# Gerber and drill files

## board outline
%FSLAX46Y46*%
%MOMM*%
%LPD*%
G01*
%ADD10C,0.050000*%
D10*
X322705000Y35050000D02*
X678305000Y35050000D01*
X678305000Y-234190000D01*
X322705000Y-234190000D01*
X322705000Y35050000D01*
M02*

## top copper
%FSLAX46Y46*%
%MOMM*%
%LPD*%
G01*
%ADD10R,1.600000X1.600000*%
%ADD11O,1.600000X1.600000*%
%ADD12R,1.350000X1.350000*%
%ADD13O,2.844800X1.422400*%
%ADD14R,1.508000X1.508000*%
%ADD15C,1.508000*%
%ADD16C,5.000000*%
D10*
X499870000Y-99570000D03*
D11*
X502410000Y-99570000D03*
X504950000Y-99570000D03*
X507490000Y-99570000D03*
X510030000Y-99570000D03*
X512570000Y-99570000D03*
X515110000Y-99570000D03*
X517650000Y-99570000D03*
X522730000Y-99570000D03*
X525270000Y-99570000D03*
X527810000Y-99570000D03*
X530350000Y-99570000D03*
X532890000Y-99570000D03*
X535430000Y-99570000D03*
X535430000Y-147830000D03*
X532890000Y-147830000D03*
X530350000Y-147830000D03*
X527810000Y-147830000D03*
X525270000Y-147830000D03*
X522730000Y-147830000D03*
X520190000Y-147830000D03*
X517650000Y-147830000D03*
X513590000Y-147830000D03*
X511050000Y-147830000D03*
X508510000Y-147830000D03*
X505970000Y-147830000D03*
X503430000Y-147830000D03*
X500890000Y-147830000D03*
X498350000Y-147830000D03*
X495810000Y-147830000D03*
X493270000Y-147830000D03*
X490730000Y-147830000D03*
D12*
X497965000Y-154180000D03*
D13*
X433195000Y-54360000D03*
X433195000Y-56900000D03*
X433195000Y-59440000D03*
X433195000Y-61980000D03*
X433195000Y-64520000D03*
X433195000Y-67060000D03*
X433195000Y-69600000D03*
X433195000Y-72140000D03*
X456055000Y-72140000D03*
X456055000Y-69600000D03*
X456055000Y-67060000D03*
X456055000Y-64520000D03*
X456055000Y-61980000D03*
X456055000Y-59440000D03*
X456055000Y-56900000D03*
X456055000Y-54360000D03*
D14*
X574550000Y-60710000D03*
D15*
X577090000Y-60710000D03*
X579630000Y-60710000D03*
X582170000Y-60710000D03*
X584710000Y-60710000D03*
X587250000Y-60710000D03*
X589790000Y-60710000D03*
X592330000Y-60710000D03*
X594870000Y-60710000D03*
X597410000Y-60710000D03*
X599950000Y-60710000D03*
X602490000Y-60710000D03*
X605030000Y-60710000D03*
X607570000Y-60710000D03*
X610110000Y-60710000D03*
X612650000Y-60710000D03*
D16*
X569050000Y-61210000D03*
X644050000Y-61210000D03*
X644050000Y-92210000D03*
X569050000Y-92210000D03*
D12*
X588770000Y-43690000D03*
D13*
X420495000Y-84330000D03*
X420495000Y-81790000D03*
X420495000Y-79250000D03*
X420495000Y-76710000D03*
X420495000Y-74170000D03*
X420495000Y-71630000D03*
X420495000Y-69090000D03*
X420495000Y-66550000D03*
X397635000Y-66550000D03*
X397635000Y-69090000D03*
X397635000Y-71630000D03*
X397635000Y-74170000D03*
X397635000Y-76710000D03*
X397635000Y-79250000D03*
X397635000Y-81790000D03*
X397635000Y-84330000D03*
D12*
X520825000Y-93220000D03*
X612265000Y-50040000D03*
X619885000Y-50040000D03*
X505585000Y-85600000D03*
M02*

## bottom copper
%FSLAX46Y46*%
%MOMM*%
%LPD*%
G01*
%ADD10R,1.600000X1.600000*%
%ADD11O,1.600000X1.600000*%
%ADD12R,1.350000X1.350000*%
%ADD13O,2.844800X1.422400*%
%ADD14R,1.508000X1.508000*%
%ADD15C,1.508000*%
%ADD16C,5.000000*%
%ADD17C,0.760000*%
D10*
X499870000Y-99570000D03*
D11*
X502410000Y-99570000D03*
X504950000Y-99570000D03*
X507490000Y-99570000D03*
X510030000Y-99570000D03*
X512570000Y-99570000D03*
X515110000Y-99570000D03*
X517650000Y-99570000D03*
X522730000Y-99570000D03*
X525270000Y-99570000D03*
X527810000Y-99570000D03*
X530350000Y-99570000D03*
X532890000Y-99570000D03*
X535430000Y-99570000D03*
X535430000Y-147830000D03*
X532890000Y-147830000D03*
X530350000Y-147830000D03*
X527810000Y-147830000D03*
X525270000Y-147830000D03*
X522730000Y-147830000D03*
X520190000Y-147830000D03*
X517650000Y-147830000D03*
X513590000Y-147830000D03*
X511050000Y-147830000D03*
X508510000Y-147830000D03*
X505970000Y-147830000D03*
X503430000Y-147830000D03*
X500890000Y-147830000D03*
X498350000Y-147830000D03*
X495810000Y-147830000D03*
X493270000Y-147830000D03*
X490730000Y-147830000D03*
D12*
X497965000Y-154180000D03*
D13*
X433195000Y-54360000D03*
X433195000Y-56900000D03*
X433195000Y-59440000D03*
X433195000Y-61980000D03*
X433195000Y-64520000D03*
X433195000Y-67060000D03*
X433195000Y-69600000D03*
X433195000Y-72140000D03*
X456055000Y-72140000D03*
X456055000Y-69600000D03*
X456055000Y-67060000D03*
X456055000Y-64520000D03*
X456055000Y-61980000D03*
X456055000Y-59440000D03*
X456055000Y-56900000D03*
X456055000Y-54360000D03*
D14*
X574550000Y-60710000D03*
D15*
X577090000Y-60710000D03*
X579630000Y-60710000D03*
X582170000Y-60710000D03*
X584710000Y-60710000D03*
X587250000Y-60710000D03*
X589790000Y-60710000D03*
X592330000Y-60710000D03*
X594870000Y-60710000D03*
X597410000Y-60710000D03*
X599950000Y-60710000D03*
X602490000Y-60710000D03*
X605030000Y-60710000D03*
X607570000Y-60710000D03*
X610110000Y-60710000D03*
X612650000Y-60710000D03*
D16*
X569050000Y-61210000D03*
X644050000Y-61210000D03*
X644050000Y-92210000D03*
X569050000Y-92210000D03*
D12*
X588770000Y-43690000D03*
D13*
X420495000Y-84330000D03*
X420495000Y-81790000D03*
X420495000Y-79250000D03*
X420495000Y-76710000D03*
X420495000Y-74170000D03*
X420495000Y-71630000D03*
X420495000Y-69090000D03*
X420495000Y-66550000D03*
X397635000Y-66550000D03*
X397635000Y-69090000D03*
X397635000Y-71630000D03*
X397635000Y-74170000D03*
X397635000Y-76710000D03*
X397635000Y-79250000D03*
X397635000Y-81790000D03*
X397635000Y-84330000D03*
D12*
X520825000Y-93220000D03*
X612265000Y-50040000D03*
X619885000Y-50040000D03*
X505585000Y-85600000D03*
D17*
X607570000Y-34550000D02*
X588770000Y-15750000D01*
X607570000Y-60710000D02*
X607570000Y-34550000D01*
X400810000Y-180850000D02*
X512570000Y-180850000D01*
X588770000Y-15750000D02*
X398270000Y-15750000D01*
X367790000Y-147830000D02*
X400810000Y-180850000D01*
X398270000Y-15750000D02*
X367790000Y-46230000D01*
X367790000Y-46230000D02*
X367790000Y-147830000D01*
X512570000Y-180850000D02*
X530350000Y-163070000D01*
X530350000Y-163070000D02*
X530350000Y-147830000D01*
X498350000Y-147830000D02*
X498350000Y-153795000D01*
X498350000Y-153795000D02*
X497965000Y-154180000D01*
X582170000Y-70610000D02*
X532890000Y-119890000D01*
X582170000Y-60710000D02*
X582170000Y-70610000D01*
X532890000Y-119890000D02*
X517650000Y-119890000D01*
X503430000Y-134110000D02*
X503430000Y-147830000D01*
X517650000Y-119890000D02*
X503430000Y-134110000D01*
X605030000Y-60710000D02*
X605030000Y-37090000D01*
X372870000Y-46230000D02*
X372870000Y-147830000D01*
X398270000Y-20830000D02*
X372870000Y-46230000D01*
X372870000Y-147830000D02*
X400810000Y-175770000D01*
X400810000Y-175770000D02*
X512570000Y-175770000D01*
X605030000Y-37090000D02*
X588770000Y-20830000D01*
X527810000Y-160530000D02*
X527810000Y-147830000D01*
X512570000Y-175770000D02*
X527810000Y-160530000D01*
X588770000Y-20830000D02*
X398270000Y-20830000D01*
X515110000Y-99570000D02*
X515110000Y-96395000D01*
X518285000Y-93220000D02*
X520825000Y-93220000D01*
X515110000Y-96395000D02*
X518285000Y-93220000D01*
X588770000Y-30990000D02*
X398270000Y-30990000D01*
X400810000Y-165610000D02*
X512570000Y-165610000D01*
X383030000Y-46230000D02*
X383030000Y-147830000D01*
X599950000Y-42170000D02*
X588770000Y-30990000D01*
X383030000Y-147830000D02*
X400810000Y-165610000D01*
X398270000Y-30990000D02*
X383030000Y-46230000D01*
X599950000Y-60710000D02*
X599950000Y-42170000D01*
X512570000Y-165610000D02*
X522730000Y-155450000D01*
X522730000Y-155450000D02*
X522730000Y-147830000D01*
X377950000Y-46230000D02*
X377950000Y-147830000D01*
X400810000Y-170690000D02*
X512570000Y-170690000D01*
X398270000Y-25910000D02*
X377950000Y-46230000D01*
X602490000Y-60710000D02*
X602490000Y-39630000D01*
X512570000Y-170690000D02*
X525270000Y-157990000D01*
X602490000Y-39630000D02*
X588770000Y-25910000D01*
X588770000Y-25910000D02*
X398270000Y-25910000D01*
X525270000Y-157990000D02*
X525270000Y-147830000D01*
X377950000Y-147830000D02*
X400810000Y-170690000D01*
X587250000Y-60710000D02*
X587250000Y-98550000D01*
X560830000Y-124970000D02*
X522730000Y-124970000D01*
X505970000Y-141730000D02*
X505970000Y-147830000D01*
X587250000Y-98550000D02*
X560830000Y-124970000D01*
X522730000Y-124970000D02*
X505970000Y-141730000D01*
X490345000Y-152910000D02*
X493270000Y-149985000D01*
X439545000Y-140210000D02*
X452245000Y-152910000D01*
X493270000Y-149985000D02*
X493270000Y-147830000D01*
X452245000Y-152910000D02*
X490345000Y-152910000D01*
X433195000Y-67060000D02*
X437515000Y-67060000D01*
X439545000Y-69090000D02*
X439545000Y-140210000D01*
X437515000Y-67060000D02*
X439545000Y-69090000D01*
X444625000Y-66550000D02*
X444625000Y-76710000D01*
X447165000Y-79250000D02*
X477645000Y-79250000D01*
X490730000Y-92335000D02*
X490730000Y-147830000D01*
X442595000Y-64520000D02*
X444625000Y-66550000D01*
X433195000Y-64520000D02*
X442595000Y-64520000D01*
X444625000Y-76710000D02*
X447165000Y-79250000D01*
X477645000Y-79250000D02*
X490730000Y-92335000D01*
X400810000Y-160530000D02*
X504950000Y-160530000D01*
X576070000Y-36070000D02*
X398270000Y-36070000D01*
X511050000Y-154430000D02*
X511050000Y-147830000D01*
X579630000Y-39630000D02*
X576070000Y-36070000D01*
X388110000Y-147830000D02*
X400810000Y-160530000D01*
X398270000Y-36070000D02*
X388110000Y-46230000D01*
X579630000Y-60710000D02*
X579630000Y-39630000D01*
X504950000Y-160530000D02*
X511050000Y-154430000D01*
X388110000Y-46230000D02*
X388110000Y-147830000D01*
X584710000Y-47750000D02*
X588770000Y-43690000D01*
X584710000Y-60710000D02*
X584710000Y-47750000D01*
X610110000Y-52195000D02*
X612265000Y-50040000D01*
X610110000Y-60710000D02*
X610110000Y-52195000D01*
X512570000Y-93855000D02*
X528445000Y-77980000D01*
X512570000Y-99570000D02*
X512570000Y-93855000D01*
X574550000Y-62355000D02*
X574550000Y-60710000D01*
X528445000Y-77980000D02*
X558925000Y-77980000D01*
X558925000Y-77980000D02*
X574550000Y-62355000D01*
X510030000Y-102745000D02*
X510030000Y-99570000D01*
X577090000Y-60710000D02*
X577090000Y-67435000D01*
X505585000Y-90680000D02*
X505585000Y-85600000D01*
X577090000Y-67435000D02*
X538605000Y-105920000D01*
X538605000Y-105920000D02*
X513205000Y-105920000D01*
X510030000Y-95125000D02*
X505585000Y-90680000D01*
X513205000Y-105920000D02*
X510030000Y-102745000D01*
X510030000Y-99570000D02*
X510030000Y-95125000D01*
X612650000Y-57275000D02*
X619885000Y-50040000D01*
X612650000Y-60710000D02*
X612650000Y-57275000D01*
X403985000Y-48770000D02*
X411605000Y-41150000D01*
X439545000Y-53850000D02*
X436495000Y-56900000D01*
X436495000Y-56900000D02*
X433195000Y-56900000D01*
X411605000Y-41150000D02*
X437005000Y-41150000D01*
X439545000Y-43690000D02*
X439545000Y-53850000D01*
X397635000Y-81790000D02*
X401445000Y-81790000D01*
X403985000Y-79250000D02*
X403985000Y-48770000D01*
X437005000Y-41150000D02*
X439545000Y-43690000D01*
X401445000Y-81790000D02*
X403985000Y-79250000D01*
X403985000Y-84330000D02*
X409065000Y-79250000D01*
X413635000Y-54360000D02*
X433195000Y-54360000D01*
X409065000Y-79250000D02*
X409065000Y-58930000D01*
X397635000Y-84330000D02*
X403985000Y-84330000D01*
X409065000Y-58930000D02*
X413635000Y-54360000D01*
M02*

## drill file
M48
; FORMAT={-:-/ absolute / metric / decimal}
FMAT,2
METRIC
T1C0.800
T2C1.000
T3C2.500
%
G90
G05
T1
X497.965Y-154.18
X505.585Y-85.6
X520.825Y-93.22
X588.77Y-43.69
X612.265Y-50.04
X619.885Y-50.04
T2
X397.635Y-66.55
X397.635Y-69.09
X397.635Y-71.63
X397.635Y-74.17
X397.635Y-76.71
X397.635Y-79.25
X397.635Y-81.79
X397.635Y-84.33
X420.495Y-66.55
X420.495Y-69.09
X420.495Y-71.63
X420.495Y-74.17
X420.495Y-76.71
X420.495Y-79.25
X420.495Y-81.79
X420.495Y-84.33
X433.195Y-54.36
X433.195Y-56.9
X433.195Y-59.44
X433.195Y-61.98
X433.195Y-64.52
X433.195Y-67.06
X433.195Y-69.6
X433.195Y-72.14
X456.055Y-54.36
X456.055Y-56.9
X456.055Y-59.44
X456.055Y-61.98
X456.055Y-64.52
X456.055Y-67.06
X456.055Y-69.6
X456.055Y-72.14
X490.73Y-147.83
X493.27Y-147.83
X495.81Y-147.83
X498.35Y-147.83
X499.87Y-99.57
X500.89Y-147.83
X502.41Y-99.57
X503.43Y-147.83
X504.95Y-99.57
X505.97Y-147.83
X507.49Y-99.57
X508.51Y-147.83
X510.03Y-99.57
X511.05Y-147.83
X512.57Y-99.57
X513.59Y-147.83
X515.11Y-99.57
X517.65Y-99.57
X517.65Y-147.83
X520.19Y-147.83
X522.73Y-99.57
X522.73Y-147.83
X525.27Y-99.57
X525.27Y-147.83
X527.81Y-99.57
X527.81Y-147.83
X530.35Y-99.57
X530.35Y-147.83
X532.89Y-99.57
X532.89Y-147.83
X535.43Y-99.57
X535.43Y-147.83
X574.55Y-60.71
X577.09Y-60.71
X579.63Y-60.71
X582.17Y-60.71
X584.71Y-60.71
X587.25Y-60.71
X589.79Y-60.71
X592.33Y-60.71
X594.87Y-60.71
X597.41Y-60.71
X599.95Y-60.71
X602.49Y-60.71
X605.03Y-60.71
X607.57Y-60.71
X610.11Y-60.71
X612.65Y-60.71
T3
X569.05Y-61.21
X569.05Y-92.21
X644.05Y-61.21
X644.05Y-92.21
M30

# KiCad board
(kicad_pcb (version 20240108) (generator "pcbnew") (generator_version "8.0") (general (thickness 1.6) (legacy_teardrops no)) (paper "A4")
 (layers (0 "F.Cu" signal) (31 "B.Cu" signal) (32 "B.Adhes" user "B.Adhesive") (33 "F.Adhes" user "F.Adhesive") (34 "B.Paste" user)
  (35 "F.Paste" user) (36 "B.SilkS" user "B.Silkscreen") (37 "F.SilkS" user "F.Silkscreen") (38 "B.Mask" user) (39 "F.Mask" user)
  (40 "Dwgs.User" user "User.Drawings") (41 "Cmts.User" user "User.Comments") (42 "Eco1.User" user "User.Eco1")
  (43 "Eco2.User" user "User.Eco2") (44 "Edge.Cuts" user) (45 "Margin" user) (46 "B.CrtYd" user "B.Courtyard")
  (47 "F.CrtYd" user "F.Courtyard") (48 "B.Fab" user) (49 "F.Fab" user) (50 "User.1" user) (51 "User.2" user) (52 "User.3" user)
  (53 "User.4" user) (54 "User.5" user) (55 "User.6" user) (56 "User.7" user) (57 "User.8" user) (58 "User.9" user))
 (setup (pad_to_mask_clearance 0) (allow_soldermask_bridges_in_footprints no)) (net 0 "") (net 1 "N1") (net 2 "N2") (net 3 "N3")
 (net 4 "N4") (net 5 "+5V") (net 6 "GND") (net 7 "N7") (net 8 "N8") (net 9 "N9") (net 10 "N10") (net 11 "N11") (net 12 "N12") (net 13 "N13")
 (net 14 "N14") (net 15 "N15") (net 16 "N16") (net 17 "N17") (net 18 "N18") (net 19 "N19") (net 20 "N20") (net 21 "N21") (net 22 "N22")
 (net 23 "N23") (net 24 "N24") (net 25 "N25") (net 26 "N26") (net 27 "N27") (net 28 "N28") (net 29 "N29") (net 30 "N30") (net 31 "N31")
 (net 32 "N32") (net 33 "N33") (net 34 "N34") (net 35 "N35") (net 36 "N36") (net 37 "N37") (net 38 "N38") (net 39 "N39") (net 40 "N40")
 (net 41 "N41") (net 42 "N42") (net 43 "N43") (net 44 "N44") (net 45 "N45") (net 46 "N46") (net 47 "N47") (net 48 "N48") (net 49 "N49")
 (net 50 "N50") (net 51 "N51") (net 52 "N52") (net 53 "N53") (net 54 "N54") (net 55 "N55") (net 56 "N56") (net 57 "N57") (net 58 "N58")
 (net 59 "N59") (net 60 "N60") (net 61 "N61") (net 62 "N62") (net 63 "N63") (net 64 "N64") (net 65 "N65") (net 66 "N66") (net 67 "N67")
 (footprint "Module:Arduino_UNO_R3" (layer "F.Cu") (at 499.87 99.57)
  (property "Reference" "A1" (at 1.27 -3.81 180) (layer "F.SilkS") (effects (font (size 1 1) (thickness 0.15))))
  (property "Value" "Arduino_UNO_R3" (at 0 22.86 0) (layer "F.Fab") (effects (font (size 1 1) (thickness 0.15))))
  (pad "1" thru_hole rect (at 0 0 90) (size 1.6 1.6) (drill 1) (layers "*.Cu" "*.Mask") (remove_unused_layers no) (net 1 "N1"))
  (pad "2" thru_hole oval (at 2.54 0 90) (size 1.6 1.6) (drill 1) (layers "*.Cu" "*.Mask") (remove_unused_layers no) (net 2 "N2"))
  (pad "3" thru_hole oval (at 5.08 0 90) (size 1.6 1.6) (drill 1) (layers "*.Cu" "*.Mask") (remove_unused_layers no) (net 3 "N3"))
  (pad "4" thru_hole oval (at 7.62 0 90) (size 1.6 1.6) (drill 1) (layers "*.Cu" "*.Mask") (remove_unused_layers no) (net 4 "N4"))
  (pad "5" thru_hole oval (at 10.16 0 90) (size 1.6 1.6) (drill 1) (layers "*.Cu" "*.Mask") (remove_unused_layers no) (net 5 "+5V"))
  (pad "6" thru_hole oval (at 12.7 0 90) (size 1.6 1.6) (drill 1) (layers "*.Cu" "*.Mask") (remove_unused_layers no) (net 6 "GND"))
  (pad "7" thru_hole oval (at 15.24 0 90) (size 1.6 1.6) (drill 1) (layers "*.Cu" "*.Mask") (remove_unused_layers no) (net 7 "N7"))
  (pad "8" thru_hole oval (at 17.78 0 90) (size 1.6 1.6) (drill 1) (layers "*.Cu" "*.Mask") (remove_unused_layers no) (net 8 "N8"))
  (pad "9" thru_hole oval (at 22.86 0 90) (size 1.6 1.6) (drill 1) (layers "*.Cu" "*.Mask") (remove_unused_layers no) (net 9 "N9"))
  (pad "10" thru_hole oval (at 25.4 0 90) (size 1.6 1.6) (drill 1) (layers "*.Cu" "*.Mask") (remove_unused_layers no) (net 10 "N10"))
  (pad "11" thru_hole oval (at 27.94 0 90) (size 1.6 1.6) (drill 1) (layers "*.Cu" "*.Mask") (remove_unused_layers no) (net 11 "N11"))
  (pad "12" thru_hole oval (at 30.48 0 90) (size 1.6 1.6) (drill 1) (layers "*.Cu" "*.Mask") (remove_unused_layers no) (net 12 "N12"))
  (pad "13" thru_hole oval (at 33.02 0 90) (size 1.6 1.6) (drill 1) (layers "*.Cu" "*.Mask") (remove_unused_layers no) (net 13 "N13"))
  (pad "14" thru_hole oval (at 35.56 0 90) (size 1.6 1.6) (drill 1) (layers "*.Cu" "*.Mask") (remove_unused_layers no) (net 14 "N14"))
  (pad "15" thru_hole oval (at 35.56 48.26 90) (size 1.6 1.6) (drill 1) (layers "*.Cu" "*.Mask") (remove_unused_layers no) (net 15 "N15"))
  (pad "16" thru_hole oval (at 33.02 48.26 90) (size 1.6 1.6) (drill 1) (layers "*.Cu" "*.Mask") (remove_unused_layers no) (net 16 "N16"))
  (pad "17" thru_hole oval (at 30.48 48.26 90) (size 1.6 1.6) (drill 1) (layers "*.Cu" "*.Mask") (remove_unused_layers no) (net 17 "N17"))
  (pad "18" thru_hole oval (at 27.94 48.26 90) (size 1.6 1.6) (drill 1) (layers "*.Cu" "*.Mask") (remove_unused_layers no) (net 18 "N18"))
  (pad "19" thru_hole oval (at 25.4 48.26 90) (size 1.6 1.6) (drill 1) (layers "*.Cu" "*.Mask") (remove_unused_layers no) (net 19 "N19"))
  (pad "20" thru_hole oval (at 22.86 48.26 90) (size 1.6 1.6) (drill 1) (layers "*.Cu" "*.Mask") (remove_unused_layers no) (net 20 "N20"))
  (pad "21" thru_hole oval (at 20.32 48.26 90) (size 1.6 1.6) (drill 1) (layers "*.Cu" "*.Mask") (remove_unused_layers no) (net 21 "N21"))
  (pad "22" thru_hole oval (at 17.78 48.26 90) (size 1.6 1.6) (drill 1) (layers "*.Cu" "*.Mask") (remove_unused_layers no) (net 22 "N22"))
  (pad "23" thru_hole oval (at 13.72 48.26 90) (size 1.6 1.6) (drill 1) (layers "*.Cu" "*.Mask") (remove_unused_layers no) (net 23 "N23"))
  (pad "24" thru_hole oval (at 11.18 48.26 90) (size 1.6 1.6) (drill 1) (layers "*.Cu" "*.Mask") (remove_unused_layers no) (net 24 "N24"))
  (pad "25" thru_hole oval (at 8.64 48.26 90) (size 1.6 1.6) (drill 1) (layers "*.Cu" "*.Mask") (remove_unused_layers no) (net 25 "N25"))
  (pad "26" thru_hole oval (at 6.1 48.26 90) (size 1.6 1.6) (drill 1) (layers "*.Cu" "*.Mask") (remove_unused_layers no) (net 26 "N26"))
  (pad "27" thru_hole oval (at 3.56 48.26 90) (size 1.6 1.6) (drill 1) (layers "*.Cu" "*.Mask") (remove_unused_layers no) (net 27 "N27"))
  (pad "28" thru_hole oval (at 1.02 48.26 90) (size 1.6 1.6) (drill 1) (layers "*.Cu" "*.Mask") (remove_unused_layers no) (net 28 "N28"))
  (pad "29" thru_hole oval (at -1.52 48.26 90) (size 1.6 1.6) (drill 1) (layers "*.Cu" "*.Mask") (remove_unused_layers no) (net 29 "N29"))
  (pad "30" thru_hole oval (at -4.06 48.26 90) (size 1.6 1.6) (drill 1) (layers "*.Cu" "*.Mask") (remove_unused_layers no) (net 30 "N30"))
  (pad "31" thru_hole oval (at -6.6 48.26 90) (size 1.6 1.6) (drill 1) (layers "*.Cu" "*.Mask") (remove_unused_layers no) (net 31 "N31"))
  (pad "32" thru_hole oval (at -9.14 48.26 90) (size 1.6 1.6) (drill 1) (layers "*.Cu" "*.Mask") (remove_unused_layers no) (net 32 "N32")))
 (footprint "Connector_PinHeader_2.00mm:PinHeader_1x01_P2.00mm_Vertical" (layer "F.Cu") (at 497.965 154.18)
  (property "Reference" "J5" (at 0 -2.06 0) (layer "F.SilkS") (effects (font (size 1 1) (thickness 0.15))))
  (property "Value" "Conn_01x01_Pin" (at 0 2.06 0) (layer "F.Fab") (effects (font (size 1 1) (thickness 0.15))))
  (pad "1" thru_hole rect (at 0 0) (size 1.35 1.35) (drill 0.8) (layers "*.Cu" "*.Mask") (remove_unused_layers no) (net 29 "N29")))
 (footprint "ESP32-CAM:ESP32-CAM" (layer "F.Cu") (at 444.625 64.52)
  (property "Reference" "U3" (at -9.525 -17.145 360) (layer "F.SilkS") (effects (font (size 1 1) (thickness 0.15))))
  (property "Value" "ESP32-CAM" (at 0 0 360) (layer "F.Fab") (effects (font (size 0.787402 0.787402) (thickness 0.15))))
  (pad "P$1" thru_hole oval (at -11.43 -10.16) (size 2.8448 1.4224) (drill 1) (layers "*.Cu" "*.Mask") (remove_unused_layers no)
   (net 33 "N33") (solder_mask_margin 0.102))
  (pad "P$2" thru_hole oval (at -11.43 -7.62) (size 2.8448 1.4224) (drill 1) (layers "*.Cu" "*.Mask") (remove_unused_layers no)
   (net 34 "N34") (solder_mask_margin 0.102))
  (pad "P$3" thru_hole oval (at -11.43 -5.08) (size 2.8448 1.4224) (drill 1) (layers "*.Cu" "*.Mask") (remove_unused_layers no)
   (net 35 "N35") (solder_mask_margin 0.102))
  (pad "P$4" thru_hole oval (at -11.43 -2.54) (size 2.8448 1.4224) (drill 1) (layers "*.Cu" "*.Mask") (remove_unused_layers no)
   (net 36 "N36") (solder_mask_margin 0.102))
  (pad "P$5" thru_hole oval (at -11.43 0) (size 2.8448 1.4224) (drill 1) (layers "*.Cu" "*.Mask") (remove_unused_layers no) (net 32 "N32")
   (solder_mask_margin 0.102))
  (pad "P$6" thru_hole oval (at -11.43 2.54) (size 2.8448 1.4224) (drill 1) (layers "*.Cu" "*.Mask") (remove_unused_layers no)
   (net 31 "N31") (solder_mask_margin 0.102))
  (pad "P$7" thru_hole oval (at -11.43 5.08) (size 2.8448 1.4224) (drill 1) (layers "*.Cu" "*.Mask") (remove_unused_layers no)
   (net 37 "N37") (solder_mask_margin 0.102))
  (pad "P$8" thru_hole oval (at -11.43 7.62) (size 2.8448 1.4224) (drill 1) (layers "*.Cu" "*.Mask") (remove_unused_layers no)
   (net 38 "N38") (solder_mask_margin 0.102))
  (pad "P$9" thru_hole oval (at 11.43 7.62) (size 2.8448 1.4224) (drill 1) (layers "*.Cu" "*.Mask") (remove_unused_layers no) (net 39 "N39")
   (solder_mask_margin 0.102))
  (pad "P$10" thru_hole oval (at 11.43 5.08) (size 2.8448 1.4224) (drill 1) (layers "*.Cu" "*.Mask") (remove_unused_layers no)
   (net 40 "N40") (solder_mask_margin 0.102))
  (pad "P$11" thru_hole oval (at 11.43 2.54) (size 2.8448 1.4224) (drill 1) (layers "*.Cu" "*.Mask") (remove_unused_layers no)
   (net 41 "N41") (solder_mask_margin 0.102))
  (pad "P$12" thru_hole oval (at 11.43 0) (size 2.8448 1.4224) (drill 1) (layers "*.Cu" "*.Mask") (remove_unused_layers no) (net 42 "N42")
   (solder_mask_margin 0.102))
  (pad "P$13" thru_hole oval (at 11.43 -2.54) (size 2.8448 1.4224) (drill 1) (layers "*.Cu" "*.Mask") (remove_unused_layers no)
   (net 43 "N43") (solder_mask_margin 0.102))
  (pad "P$14" thru_hole oval (at 11.43 -5.08) (size 2.8448 1.4224) (drill 1) (layers "*.Cu" "*.Mask") (remove_unused_layers no)
   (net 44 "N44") (solder_mask_margin 0.102))
  (pad "P$15" thru_hole oval (at 11.43 -7.62) (size 2.8448 1.4224) (drill 1) (layers "*.Cu" "*.Mask") (remove_unused_layers no)
   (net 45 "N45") (solder_mask_margin 0.102))
  (pad "P$16" thru_hole oval (at 11.43 -10.16) (size 2.8448 1.4224) (drill 1) (layers "*.Cu" "*.Mask") (remove_unused_layers no)
   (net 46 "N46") (solder_mask_margin 0.102)))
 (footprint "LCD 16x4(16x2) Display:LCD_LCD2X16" (layer "F.Cu") (at 606.55 76.71)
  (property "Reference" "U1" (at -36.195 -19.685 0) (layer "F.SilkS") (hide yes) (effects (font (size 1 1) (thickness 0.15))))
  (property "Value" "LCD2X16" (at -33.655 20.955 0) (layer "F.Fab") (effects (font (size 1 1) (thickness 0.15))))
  (pad "1" thru_hole rect (at -32 -16) (size 1.508 1.508) (drill 1) (layers "*.Cu" "*.Mask") (remove_unused_layers no) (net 6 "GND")
   (solder_mask_margin 0.102))
  (pad "2" thru_hole circle (at -29.46 -16) (size 1.508 1.508) (drill 1) (layers "*.Cu" "*.Mask") (remove_unused_layers no) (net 5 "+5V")
   (solder_mask_margin 0.102))
  (pad "3" thru_hole circle (at -26.92 -16) (size 1.508 1.508) (drill 1) (layers "*.Cu" "*.Mask") (remove_unused_layers no) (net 24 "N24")
   (solder_mask_margin 0.102))
  (pad "4" thru_hole circle (at -24.38 -16) (size 1.508 1.508) (drill 1) (layers "*.Cu" "*.Mask") (remove_unused_layers no) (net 27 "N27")
   (solder_mask_margin 0.102))
  (pad "5" thru_hole circle (at -21.84 -16) (size 1.508 1.508) (drill 1) (layers "*.Cu" "*.Mask") (remove_unused_layers no) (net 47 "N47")
   (solder_mask_margin 0.102))
  (pad "6" thru_hole circle (at -19.3 -16) (size 1.508 1.508) (drill 1) (layers "*.Cu" "*.Mask") (remove_unused_layers no) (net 26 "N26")
   (solder_mask_margin 0.102))
  (pad "7" thru_hole circle (at -16.76 -16) (size 1.508 1.508) (drill 1) (layers "*.Cu" "*.Mask") (remove_unused_layers no) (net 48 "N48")
   (solder_mask_margin 0.102))
  (pad "8" thru_hole circle (at -14.22 -16) (size 1.508 1.508) (drill 1) (layers "*.Cu" "*.Mask") (remove_unused_layers no) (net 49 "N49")
   (solder_mask_margin 0.102))
  (pad "9" thru_hole circle (at -11.68 -16) (size 1.508 1.508) (drill 1) (layers "*.Cu" "*.Mask") (remove_unused_layers no) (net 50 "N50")
   (solder_mask_margin 0.102))
  (pad "10" thru_hole circle (at -9.14 -16) (size 1.508 1.508) (drill 1) (layers "*.Cu" "*.Mask") (remove_unused_layers no) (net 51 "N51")
   (solder_mask_margin 0.102))
  (pad "11" thru_hole circle (at -6.6 -16) (size 1.508 1.508) (drill 1) (layers "*.Cu" "*.Mask") (remove_unused_layers no) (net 20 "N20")
   (solder_mask_margin 0.102))
  (pad "12" thru_hole circle (at -4.06 -16) (size 1.508 1.508) (drill 1) (layers "*.Cu" "*.Mask") (remove_unused_layers no) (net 19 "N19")
   (solder_mask_margin 0.102))
  (pad "13" thru_hole circle (at -1.52 -16) (size 1.508 1.508) (drill 1) (layers "*.Cu" "*.Mask") (remove_unused_layers no) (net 18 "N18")
   (solder_mask_margin 0.102))
  (pad "14" thru_hole circle (at 1.02 -16) (size 1.508 1.508) (drill 1) (layers "*.Cu" "*.Mask") (remove_unused_layers no) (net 17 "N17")
   (solder_mask_margin 0.102))
  (pad "15" thru_hole circle (at 3.56 -16) (size 1.508 1.508) (drill 1) (layers "*.Cu" "*.Mask") (remove_unused_layers no) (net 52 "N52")
   (solder_mask_margin 0.102))
  (pad "16" thru_hole circle (at 6.1 -16) (size 1.508 1.508) (drill 1) (layers "*.Cu" "*.Mask") (remove_unused_layers no) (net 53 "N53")
   (solder_mask_margin 0.102))
  (pad "S1" thru_hole circle (at -37.5 -15.5) (size 5 5) (drill 2.5) (layers "*.Cu" "*.Mask") (remove_unused_layers no)
   (solder_mask_margin 0.102))
  (pad "S2" thru_hole circle (at 37.5 -15.5) (size 5 5) (drill 2.5) (layers "*.Cu" "*.Mask") (remove_unused_layers no)
   (solder_mask_margin 0.102))
  (pad "S3" thru_hole circle (at 37.5 15.5) (size 5 5) (drill 2.5) (layers "*.Cu" "*.Mask") (remove_unused_layers no)
   (solder_mask_margin 0.102))
  (pad "S4" thru_hole circle (at -37.5 15.5) (size 5 5) (drill 2.5) (layers "*.Cu" "*.Mask") (remove_unused_layers no)
   (solder_mask_margin 0.102)))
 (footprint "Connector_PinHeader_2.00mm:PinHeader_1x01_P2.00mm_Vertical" (layer "F.Cu") (at 588.77 43.69)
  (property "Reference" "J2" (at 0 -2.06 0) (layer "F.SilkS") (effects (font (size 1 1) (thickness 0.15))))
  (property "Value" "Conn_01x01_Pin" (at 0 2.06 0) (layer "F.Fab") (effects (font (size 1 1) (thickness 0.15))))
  (pad "1" thru_hole rect (at 0 0) (size 1.35 1.35) (drill 0.8) (layers "*.Cu" "*.Mask") (remove_unused_layers no) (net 47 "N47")))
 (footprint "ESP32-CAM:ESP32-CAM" (layer "F.Cu") (at 409.065 74.17 180)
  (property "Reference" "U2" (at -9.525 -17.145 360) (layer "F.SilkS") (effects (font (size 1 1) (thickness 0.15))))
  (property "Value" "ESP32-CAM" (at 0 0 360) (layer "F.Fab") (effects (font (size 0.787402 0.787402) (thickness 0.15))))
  (pad "P$1" thru_hole oval (at -11.43 -10.16 180) (size 2.8448 1.4224) (drill 1) (layers "*.Cu" "*.Mask") (remove_unused_layers no)
   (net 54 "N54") (solder_mask_margin 0.102))
  (pad "P$2" thru_hole oval (at -11.43 -7.62 180) (size 2.8448 1.4224) (drill 1) (layers "*.Cu" "*.Mask") (remove_unused_layers no)
   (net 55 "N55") (solder_mask_margin 0.102))
  (pad "P$3" thru_hole oval (at -11.43 -5.08 180) (size 2.8448 1.4224) (drill 1) (layers "*.Cu" "*.Mask") (remove_unused_layers no)
   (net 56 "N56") (solder_mask_margin 0.102))
  (pad "P$4" thru_hole oval (at -11.43 -2.54 180) (size 2.8448 1.4224) (drill 1) (layers "*.Cu" "*.Mask") (remove_unused_layers no)
   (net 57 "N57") (solder_mask_margin 0.102))
  (pad "P$5" thru_hole oval (at -11.43 0 180) (size 2.8448 1.4224) (drill 1) (layers "*.Cu" "*.Mask") (remove_unused_layers no)
   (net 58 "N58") (solder_mask_margin 0.102))
  (pad "P$6" thru_hole oval (at -11.43 2.54 180) (size 2.8448 1.4224) (drill 1) (layers "*.Cu" "*.Mask") (remove_unused_layers no)
   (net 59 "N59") (solder_mask_margin 0.102))
  (pad "P$7" thru_hole oval (at -11.43 5.08 180) (size 2.8448 1.4224) (drill 1) (layers "*.Cu" "*.Mask") (remove_unused_layers no)
   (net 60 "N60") (solder_mask_margin 0.102))
  (pad "P$8" thru_hole oval (at -11.43 7.62 180) (size 2.8448 1.4224) (drill 1) (layers "*.Cu" "*.Mask") (remove_unused_layers no)
   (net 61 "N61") (solder_mask_margin 0.102))
  (pad "P$9" thru_hole oval (at 11.43 7.62 180) (size 2.8448 1.4224) (drill 1) (layers "*.Cu" "*.Mask") (remove_unused_layers no)
   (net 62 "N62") (solder_mask_margin 0.102))
  (pad "P$10" thru_hole oval (at 11.43 5.08 180) (size 2.8448 1.4224) (drill 1) (layers "*.Cu" "*.Mask") (remove_unused_layers no)
   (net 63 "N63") (solder_mask_margin 0.102))
  (pad "P$11" thru_hole oval (at 11.43 2.54 180) (size 2.8448 1.4224) (drill 1) (layers "*.Cu" "*.Mask") (remove_unused_layers no)
   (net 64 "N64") (solder_mask_margin 0.102))
  (pad "P$12" thru_hole oval (at 11.43 0 180) (size 2.8448 1.4224) (drill 1) (layers "*.Cu" "*.Mask") (remove_unused_layers no)
   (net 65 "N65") (solder_mask_margin 0.102))
  (pad "P$13" thru_hole oval (at 11.43 -2.54 180) (size 2.8448 1.4224) (drill 1) (layers "*.Cu" "*.Mask") (remove_unused_layers no)
   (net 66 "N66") (solder_mask_margin 0.102))
  (pad "P$14" thru_hole oval (at 11.43 -5.08 180) (size 2.8448 1.4224) (drill 1) (layers "*.Cu" "*.Mask") (remove_unused_layers no)
   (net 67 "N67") (solder_mask_margin 0.102))
  (pad "P$15" thru_hole oval (at 11.43 -7.62 180) (size 2.8448 1.4224) (drill 1) (layers "*.Cu" "*.Mask") (remove_unused_layers no)
   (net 34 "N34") (solder_mask_margin 0.102))
  (pad "P$16" thru_hole oval (at 11.43 -10.16 180) (size 2.8448 1.4224) (drill 1) (layers "*.Cu" "*.Mask") (remove_unused_layers no)
   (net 33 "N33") (solder_mask_margin 0.102)))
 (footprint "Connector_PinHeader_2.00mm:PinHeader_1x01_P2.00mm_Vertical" (layer "F.Cu") (at 520.825 93.22)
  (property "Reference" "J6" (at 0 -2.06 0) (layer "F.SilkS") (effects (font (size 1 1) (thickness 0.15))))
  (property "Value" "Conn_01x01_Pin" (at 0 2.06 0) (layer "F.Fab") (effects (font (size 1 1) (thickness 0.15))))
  (pad "1" thru_hole rect (at 0 0) (size 1.35 1.35) (drill 0.8) (layers "*.Cu" "*.Mask") (remove_unused_layers no) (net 7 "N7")))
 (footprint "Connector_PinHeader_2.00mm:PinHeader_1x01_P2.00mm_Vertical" (layer "F.Cu") (at 612.265 50.04)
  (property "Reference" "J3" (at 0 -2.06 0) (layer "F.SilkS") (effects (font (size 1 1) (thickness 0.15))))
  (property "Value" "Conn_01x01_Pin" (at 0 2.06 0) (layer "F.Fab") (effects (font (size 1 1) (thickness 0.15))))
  (pad "1" thru_hole rect (at 0 0) (size 1.35 1.35) (drill 0.8) (layers "*.Cu" "*.Mask") (remove_unused_layers no) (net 52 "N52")))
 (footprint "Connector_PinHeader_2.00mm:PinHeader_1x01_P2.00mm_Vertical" (layer "F.Cu") (at 619.885 50.04)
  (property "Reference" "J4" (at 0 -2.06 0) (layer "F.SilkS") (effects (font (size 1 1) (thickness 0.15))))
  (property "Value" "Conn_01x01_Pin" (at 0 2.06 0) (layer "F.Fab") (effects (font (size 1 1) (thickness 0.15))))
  (pad "1" thru_hole rect (at 0 0) (size 1.35 1.35) (drill 0.8) (layers "*.Cu" "*.Mask") (remove_unused_layers no) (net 53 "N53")))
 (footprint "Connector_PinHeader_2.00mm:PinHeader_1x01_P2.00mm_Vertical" (layer "F.Cu") (at 505.585 85.6)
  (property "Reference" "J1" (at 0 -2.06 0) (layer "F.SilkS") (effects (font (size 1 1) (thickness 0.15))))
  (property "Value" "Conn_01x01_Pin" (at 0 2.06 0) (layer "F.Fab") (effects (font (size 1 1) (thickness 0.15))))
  (pad "1" thru_hole rect (at 0 0) (size 1.35 1.35) (drill 0.8) (layers "*.Cu" "*.Mask") (remove_unused_layers no) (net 5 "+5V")))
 (gr_rect (start 322.705 -35.05) (end 678.305 234.19) (stroke (width 0.05) (type default)) (fill none) (layer "Edge.Cuts"))
 (segment (start 607.57 34.55) (end 588.77 15.75) (width 0.76) (layer "B.Cu") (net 17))
 (segment (start 607.57 60.71) (end 607.57 34.55) (width 0.76) (layer "B.Cu") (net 17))
 (segment (start 400.81 180.85) (end 512.57 180.85) (width 0.76) (layer "B.Cu") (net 17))
 (segment (start 588.77 15.75) (end 398.27 15.75) (width 0.76) (layer "B.Cu") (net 17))
 (segment (start 367.79 147.83) (end 400.81 180.85) (width 0.76) (layer "B.Cu") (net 17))
 (segment (start 398.27 15.75) (end 367.79 46.23) (width 0.76) (layer "B.Cu") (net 17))
 (segment (start 367.79 46.23) (end 367.79 147.83) (width 0.76) (layer "B.Cu") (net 17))
 (segment (start 512.57 180.85) (end 530.35 163.07) (width 0.76) (layer "B.Cu") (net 17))
 (segment (start 530.35 163.07) (end 530.35 147.83) (width 0.76) (layer "B.Cu") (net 17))
 (segment (start 498.35 147.83) (end 498.35 153.795) (width 0.76) (layer "B.Cu") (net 29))
 (segment (start 498.35 153.795) (end 497.965 154.18) (width 0.76) (layer "B.Cu") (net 29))
 (segment (start 582.17 70.61) (end 532.89 119.89) (width 0.76) (layer "B.Cu") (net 27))
 (segment (start 582.17 60.71) (end 582.17 70.61) (width 0.76) (layer "B.Cu") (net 27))
 (segment (start 532.89 119.89) (end 517.65 119.89) (width 0.76) (layer "B.Cu") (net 27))
 (segment (start 503.43 134.11) (end 503.43 147.83) (width 0.76) (layer "B.Cu") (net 27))
 (segment (start 517.65 119.89) (end 503.43 134.11) (width 0.76) (layer "B.Cu") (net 27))
 (segment (start 605.03 60.71) (end 605.03 37.09) (width 0.76) (layer "B.Cu") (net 18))
 (segment (start 372.87 46.23) (end 372.87 147.83) (width 0.76) (layer "B.Cu") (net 18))
 (segment (start 398.27 20.83) (end 372.87 46.23) (width 0.76) (layer "B.Cu") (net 18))
 (segment (start 372.87 147.83) (end 400.81 175.77) (width 0.76) (layer "B.Cu") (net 18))
 (segment (start 400.81 175.77) (end 512.57 175.77) (width 0.76) (layer "B.Cu") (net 18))
 (segment (start 605.03 37.09) (end 588.77 20.83) (width 0.76) (layer "B.Cu") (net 18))
 (segment (start 527.81 160.53) (end 527.81 147.83) (width 0.76) (layer "B.Cu") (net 18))
 (segment (start 512.57 175.77) (end 527.81 160.53) (width 0.76) (layer "B.Cu") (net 18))
 (segment (start 588.77 20.83) (end 398.27 20.83) (width 0.76) (layer "B.Cu") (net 18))
 (segment (start 515.11 99.57) (end 515.11 96.395) (width 0.76) (layer "B.Cu") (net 7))
 (segment (start 518.285 93.22) (end 520.825 93.22) (width 0.76) (layer "B.Cu") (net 7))
 (segment (start 515.11 96.395) (end 518.285 93.22) (width 0.76) (layer "B.Cu") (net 7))
 (segment (start 588.77 30.99) (end 398.27 30.99) (width 0.76) (layer "B.Cu") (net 20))
 (segment (start 400.81 165.61) (end 512.57 165.61) (width 0.76) (layer "B.Cu") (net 20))
 (segment (start 383.03 46.23) (end 383.03 147.83) (width 0.76) (layer "B.Cu") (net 20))
 (segment (start 599.95 42.17) (end 588.77 30.99) (width 0.76) (layer "B.Cu") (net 20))
 (segment (start 383.03 147.83) (end 400.81 165.61) (width 0.76) (layer "B.Cu") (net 20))
 (segment (start 398.27 30.99) (end 383.03 46.23) (width 0.76) (layer "B.Cu") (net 20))
 (segment (start 599.95 60.71) (end 599.95 42.17) (width 0.76) (layer "B.Cu") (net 20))
 (segment (start 512.57 165.61) (end 522.73 155.45) (width 0.76) (layer "B.Cu") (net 20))
 (segment (start 522.73 155.45) (end 522.73 147.83) (width 0.76) (layer "B.Cu") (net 20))
 (segment (start 377.95 46.23) (end 377.95 147.83) (width 0.76) (layer "B.Cu") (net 19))
 (segment (start 400.81 170.69) (end 512.57 170.69) (width 0.76) (layer "B.Cu") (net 19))
 (segment (start 398.27 25.91) (end 377.95 46.23) (width 0.76) (layer "B.Cu") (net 19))
 (segment (start 602.49 60.71) (end 602.49 39.63) (width 0.76) (layer "B.Cu") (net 19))
 (segment (start 512.57 170.69) (end 525.27 157.99) (width 0.76) (layer "B.Cu") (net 19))
 (segment (start 602.49 39.63) (end 588.77 25.91) (width 0.76) (layer "B.Cu") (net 19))
 (segment (start 588.77 25.91) (end 398.27 25.91) (width 0.76) (layer "B.Cu") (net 19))
 (segment (start 525.27 157.99) (end 525.27 147.83) (width 0.76) (layer "B.Cu") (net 19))
 (segment (start 377.95 147.83) (end 400.81 170.69) (width 0.76) (layer "B.Cu") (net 19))
 (segment (start 587.25 60.71) (end 587.25 98.55) (width 0.76) (layer "B.Cu") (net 26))
 (segment (start 560.83 124.97) (end 522.73 124.97) (width 0.76) (layer "B.Cu") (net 26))
 (segment (start 505.97 141.73) (end 505.97 147.83) (width 0.76) (layer "B.Cu") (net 26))
 (segment (start 587.25 98.55) (end 560.83 124.97) (width 0.76) (layer "B.Cu") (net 26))
 (segment (start 522.73 124.97) (end 505.97 141.73) (width 0.76) (layer "B.Cu") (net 26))
 (segment (start 490.345 152.91) (end 493.27 149.985) (width 0.76) (layer "B.Cu") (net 31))
 (segment (start 439.545 140.21) (end 452.245 152.91) (width 0.76) (layer "B.Cu") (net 31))
 (segment (start 493.27 149.985) (end 493.27 147.83) (width 0.76) (layer "B.Cu") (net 31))
 (segment (start 452.245 152.91) (end 490.345 152.91) (width 0.76) (layer "B.Cu") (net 31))
 (segment (start 433.195 67.06) (end 437.515 67.06) (width 0.76) (layer "B.Cu") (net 31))
 (segment (start 439.545 69.09) (end 439.545 140.21) (width 0.76) (layer "B.Cu") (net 31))
 (segment (start 437.515 67.06) (end 439.545 69.09) (width 0.76) (layer "B.Cu") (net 31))
 (segment (start 444.625 66.55) (end 444.625 76.71) (width 0.76) (layer "B.Cu") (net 32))
 (segment (start 447.165 79.25) (end 477.645 79.25) (width 0.76) (layer "B.Cu") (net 32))
 (segment (start 490.73 92.335) (end 490.73 147.83) (width 0.76) (layer "B.Cu") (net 32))
 (segment (start 442.595 64.52) (end 444.625 66.55) (width 0.76) (layer "B.Cu") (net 32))
 (segment (start 433.195 64.52) (end 442.595 64.52) (width 0.76) (layer "B.Cu") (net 32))
 (segment (start 444.625 76.71) (end 447.165 79.25) (width 0.76) (layer "B.Cu") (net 32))
 (segment (start 477.645 79.25) (end 490.73 92.335) (width 0.76) (layer "B.Cu") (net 32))
 (segment (start 400.81 160.53) (end 504.95 160.53) (width 0.76) (layer "B.Cu") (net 24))
 (segment (start 576.07 36.07) (end 398.27 36.07) (width 0.76) (layer "B.Cu") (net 24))
 (segment (start 511.05 154.43) (end 511.05 147.83) (width 0.76) (layer "B.Cu") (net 24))
 (segment (start 579.63 39.63) (end 576.07 36.07) (width 0.76) (layer "B.Cu") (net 24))
 (segment (start 388.11 147.83) (end 400.81 160.53) (width 0.76) (layer "B.Cu") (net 24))
 (segment (start 398.27 36.07) (end 388.11 46.23) (width 0.76) (layer "B.Cu") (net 24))
 (segment (start 579.63 60.71) (end 579.63 39.63) (width 0.76) (layer "B.Cu") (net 24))
 (segment (start 504.95 160.53) (end 511.05 154.43) (width 0.76) (layer "B.Cu") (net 24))
 (segment (start 388.11 46.23) (end 388.11 147.83) (width 0.76) (layer "B.Cu") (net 24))
 (segment (start 584.71 47.75) (end 588.77 43.69) (width 0.76) (layer "B.Cu") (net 47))
 (segment (start 584.71 60.71) (end 584.71 47.75) (width 0.76) (layer "B.Cu") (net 47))
 (segment (start 610.11 52.195) (end 612.265 50.04) (width 0.76) (layer "B.Cu") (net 52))
 (segment (start 610.11 60.71) (end 610.11 52.195) (width 0.76) (layer "B.Cu") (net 52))
 (segment (start 512.57 93.855) (end 528.445 77.98) (width 0.76) (layer "B.Cu") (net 6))
 (segment (start 512.57 99.57) (end 512.57 93.855) (width 0.76) (layer "B.Cu") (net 6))
 (segment (start 574.55 62.355) (end 574.55 60.71) (width 0.76) (layer "B.Cu") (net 6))
 (segment (start 528.445 77.98) (end 558.925 77.98) (width 0.76) (layer "B.Cu") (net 6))
 (segment (start 558.925 77.98) (end 574.55 62.355) (width 0.76) (layer "B.Cu") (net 6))
 (segment (start 510.03 102.745) (end 510.03 99.57) (width 0.76) (layer "B.Cu") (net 5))
 (segment (start 577.09 60.71) (end 577.09 67.435) (width 0.76) (layer "B.Cu") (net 5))
 (segment (start 505.585 90.68) (end 505.585 85.6) (width 0.76) (layer "B.Cu") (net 5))
 (segment (start 577.09 67.435) (end 538.605 105.92) (width 0.76) (layer "B.Cu") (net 5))
 (segment (start 538.605 105.92) (end 513.205 105.92) (width 0.76) (layer "B.Cu") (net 5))
 (segment (start 510.03 95.125) (end 505.585 90.68) (width 0.76) (layer "B.Cu") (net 5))
 (segment (start 513.205 105.92) (end 510.03 102.745) (width 0.76) (layer "B.Cu") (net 5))
 (segment (start 510.03 99.57) (end 510.03 95.125) (width 0.76) (layer "B.Cu") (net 5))
 (segment (start 612.65 57.275) (end 619.885 50.04) (width 0.76) (layer "B.Cu") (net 53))
 (segment (start 612.65 60.71) (end 612.65 57.275) (width 0.76) (layer "B.Cu") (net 53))
 (segment (start 403.985 48.77) (end 411.605 41.15) (width 0.76) (layer "B.Cu") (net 34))
 (segment (start 439.545 53.85) (end 436.495 56.9) (width 0.76) (layer "B.Cu") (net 34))
 (segment (start 436.495 56.9) (end 433.195 56.9) (width 0.76) (layer "B.Cu") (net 34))
 (segment (start 411.605 41.15) (end 437.005 41.15) (width 0.76) (layer "B.Cu") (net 34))
 (segment (start 439.545 43.69) (end 439.545 53.85) (width 0.76) (layer "B.Cu") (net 34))
 (segment (start 397.635 81.79) (end 401.445 81.79) (width 0.76) (layer "B.Cu") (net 34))
 (segment (start 403.985 79.25) (end 403.985 48.77) (width 0.76) (layer "B.Cu") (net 34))
 (segment (start 437.005 41.15) (end 439.545 43.69) (width 0.76) (layer "B.Cu") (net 34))
 (segment (start 401.445 81.79) (end 403.985 79.25) (width 0.76) (layer "B.Cu") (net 34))
 (segment (start 403.985 84.33) (end 409.065 79.25) (width 0.76) (layer "B.Cu") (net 33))
 (segment (start 413.635 54.36) (end 433.195 54.36) (width 0.76) (layer "B.Cu") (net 33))
 (segment (start 409.065 79.25) (end 409.065 58.93) (width 0.76) (layer "B.Cu") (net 33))
 (segment (start 397.635 84.33) (end 403.985 84.33) (width 0.76) (layer "B.Cu") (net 33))
 (segment (start 409.065 58.93) (end 413.635 54.36) (width 0.76) (layer "B.Cu") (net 33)))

